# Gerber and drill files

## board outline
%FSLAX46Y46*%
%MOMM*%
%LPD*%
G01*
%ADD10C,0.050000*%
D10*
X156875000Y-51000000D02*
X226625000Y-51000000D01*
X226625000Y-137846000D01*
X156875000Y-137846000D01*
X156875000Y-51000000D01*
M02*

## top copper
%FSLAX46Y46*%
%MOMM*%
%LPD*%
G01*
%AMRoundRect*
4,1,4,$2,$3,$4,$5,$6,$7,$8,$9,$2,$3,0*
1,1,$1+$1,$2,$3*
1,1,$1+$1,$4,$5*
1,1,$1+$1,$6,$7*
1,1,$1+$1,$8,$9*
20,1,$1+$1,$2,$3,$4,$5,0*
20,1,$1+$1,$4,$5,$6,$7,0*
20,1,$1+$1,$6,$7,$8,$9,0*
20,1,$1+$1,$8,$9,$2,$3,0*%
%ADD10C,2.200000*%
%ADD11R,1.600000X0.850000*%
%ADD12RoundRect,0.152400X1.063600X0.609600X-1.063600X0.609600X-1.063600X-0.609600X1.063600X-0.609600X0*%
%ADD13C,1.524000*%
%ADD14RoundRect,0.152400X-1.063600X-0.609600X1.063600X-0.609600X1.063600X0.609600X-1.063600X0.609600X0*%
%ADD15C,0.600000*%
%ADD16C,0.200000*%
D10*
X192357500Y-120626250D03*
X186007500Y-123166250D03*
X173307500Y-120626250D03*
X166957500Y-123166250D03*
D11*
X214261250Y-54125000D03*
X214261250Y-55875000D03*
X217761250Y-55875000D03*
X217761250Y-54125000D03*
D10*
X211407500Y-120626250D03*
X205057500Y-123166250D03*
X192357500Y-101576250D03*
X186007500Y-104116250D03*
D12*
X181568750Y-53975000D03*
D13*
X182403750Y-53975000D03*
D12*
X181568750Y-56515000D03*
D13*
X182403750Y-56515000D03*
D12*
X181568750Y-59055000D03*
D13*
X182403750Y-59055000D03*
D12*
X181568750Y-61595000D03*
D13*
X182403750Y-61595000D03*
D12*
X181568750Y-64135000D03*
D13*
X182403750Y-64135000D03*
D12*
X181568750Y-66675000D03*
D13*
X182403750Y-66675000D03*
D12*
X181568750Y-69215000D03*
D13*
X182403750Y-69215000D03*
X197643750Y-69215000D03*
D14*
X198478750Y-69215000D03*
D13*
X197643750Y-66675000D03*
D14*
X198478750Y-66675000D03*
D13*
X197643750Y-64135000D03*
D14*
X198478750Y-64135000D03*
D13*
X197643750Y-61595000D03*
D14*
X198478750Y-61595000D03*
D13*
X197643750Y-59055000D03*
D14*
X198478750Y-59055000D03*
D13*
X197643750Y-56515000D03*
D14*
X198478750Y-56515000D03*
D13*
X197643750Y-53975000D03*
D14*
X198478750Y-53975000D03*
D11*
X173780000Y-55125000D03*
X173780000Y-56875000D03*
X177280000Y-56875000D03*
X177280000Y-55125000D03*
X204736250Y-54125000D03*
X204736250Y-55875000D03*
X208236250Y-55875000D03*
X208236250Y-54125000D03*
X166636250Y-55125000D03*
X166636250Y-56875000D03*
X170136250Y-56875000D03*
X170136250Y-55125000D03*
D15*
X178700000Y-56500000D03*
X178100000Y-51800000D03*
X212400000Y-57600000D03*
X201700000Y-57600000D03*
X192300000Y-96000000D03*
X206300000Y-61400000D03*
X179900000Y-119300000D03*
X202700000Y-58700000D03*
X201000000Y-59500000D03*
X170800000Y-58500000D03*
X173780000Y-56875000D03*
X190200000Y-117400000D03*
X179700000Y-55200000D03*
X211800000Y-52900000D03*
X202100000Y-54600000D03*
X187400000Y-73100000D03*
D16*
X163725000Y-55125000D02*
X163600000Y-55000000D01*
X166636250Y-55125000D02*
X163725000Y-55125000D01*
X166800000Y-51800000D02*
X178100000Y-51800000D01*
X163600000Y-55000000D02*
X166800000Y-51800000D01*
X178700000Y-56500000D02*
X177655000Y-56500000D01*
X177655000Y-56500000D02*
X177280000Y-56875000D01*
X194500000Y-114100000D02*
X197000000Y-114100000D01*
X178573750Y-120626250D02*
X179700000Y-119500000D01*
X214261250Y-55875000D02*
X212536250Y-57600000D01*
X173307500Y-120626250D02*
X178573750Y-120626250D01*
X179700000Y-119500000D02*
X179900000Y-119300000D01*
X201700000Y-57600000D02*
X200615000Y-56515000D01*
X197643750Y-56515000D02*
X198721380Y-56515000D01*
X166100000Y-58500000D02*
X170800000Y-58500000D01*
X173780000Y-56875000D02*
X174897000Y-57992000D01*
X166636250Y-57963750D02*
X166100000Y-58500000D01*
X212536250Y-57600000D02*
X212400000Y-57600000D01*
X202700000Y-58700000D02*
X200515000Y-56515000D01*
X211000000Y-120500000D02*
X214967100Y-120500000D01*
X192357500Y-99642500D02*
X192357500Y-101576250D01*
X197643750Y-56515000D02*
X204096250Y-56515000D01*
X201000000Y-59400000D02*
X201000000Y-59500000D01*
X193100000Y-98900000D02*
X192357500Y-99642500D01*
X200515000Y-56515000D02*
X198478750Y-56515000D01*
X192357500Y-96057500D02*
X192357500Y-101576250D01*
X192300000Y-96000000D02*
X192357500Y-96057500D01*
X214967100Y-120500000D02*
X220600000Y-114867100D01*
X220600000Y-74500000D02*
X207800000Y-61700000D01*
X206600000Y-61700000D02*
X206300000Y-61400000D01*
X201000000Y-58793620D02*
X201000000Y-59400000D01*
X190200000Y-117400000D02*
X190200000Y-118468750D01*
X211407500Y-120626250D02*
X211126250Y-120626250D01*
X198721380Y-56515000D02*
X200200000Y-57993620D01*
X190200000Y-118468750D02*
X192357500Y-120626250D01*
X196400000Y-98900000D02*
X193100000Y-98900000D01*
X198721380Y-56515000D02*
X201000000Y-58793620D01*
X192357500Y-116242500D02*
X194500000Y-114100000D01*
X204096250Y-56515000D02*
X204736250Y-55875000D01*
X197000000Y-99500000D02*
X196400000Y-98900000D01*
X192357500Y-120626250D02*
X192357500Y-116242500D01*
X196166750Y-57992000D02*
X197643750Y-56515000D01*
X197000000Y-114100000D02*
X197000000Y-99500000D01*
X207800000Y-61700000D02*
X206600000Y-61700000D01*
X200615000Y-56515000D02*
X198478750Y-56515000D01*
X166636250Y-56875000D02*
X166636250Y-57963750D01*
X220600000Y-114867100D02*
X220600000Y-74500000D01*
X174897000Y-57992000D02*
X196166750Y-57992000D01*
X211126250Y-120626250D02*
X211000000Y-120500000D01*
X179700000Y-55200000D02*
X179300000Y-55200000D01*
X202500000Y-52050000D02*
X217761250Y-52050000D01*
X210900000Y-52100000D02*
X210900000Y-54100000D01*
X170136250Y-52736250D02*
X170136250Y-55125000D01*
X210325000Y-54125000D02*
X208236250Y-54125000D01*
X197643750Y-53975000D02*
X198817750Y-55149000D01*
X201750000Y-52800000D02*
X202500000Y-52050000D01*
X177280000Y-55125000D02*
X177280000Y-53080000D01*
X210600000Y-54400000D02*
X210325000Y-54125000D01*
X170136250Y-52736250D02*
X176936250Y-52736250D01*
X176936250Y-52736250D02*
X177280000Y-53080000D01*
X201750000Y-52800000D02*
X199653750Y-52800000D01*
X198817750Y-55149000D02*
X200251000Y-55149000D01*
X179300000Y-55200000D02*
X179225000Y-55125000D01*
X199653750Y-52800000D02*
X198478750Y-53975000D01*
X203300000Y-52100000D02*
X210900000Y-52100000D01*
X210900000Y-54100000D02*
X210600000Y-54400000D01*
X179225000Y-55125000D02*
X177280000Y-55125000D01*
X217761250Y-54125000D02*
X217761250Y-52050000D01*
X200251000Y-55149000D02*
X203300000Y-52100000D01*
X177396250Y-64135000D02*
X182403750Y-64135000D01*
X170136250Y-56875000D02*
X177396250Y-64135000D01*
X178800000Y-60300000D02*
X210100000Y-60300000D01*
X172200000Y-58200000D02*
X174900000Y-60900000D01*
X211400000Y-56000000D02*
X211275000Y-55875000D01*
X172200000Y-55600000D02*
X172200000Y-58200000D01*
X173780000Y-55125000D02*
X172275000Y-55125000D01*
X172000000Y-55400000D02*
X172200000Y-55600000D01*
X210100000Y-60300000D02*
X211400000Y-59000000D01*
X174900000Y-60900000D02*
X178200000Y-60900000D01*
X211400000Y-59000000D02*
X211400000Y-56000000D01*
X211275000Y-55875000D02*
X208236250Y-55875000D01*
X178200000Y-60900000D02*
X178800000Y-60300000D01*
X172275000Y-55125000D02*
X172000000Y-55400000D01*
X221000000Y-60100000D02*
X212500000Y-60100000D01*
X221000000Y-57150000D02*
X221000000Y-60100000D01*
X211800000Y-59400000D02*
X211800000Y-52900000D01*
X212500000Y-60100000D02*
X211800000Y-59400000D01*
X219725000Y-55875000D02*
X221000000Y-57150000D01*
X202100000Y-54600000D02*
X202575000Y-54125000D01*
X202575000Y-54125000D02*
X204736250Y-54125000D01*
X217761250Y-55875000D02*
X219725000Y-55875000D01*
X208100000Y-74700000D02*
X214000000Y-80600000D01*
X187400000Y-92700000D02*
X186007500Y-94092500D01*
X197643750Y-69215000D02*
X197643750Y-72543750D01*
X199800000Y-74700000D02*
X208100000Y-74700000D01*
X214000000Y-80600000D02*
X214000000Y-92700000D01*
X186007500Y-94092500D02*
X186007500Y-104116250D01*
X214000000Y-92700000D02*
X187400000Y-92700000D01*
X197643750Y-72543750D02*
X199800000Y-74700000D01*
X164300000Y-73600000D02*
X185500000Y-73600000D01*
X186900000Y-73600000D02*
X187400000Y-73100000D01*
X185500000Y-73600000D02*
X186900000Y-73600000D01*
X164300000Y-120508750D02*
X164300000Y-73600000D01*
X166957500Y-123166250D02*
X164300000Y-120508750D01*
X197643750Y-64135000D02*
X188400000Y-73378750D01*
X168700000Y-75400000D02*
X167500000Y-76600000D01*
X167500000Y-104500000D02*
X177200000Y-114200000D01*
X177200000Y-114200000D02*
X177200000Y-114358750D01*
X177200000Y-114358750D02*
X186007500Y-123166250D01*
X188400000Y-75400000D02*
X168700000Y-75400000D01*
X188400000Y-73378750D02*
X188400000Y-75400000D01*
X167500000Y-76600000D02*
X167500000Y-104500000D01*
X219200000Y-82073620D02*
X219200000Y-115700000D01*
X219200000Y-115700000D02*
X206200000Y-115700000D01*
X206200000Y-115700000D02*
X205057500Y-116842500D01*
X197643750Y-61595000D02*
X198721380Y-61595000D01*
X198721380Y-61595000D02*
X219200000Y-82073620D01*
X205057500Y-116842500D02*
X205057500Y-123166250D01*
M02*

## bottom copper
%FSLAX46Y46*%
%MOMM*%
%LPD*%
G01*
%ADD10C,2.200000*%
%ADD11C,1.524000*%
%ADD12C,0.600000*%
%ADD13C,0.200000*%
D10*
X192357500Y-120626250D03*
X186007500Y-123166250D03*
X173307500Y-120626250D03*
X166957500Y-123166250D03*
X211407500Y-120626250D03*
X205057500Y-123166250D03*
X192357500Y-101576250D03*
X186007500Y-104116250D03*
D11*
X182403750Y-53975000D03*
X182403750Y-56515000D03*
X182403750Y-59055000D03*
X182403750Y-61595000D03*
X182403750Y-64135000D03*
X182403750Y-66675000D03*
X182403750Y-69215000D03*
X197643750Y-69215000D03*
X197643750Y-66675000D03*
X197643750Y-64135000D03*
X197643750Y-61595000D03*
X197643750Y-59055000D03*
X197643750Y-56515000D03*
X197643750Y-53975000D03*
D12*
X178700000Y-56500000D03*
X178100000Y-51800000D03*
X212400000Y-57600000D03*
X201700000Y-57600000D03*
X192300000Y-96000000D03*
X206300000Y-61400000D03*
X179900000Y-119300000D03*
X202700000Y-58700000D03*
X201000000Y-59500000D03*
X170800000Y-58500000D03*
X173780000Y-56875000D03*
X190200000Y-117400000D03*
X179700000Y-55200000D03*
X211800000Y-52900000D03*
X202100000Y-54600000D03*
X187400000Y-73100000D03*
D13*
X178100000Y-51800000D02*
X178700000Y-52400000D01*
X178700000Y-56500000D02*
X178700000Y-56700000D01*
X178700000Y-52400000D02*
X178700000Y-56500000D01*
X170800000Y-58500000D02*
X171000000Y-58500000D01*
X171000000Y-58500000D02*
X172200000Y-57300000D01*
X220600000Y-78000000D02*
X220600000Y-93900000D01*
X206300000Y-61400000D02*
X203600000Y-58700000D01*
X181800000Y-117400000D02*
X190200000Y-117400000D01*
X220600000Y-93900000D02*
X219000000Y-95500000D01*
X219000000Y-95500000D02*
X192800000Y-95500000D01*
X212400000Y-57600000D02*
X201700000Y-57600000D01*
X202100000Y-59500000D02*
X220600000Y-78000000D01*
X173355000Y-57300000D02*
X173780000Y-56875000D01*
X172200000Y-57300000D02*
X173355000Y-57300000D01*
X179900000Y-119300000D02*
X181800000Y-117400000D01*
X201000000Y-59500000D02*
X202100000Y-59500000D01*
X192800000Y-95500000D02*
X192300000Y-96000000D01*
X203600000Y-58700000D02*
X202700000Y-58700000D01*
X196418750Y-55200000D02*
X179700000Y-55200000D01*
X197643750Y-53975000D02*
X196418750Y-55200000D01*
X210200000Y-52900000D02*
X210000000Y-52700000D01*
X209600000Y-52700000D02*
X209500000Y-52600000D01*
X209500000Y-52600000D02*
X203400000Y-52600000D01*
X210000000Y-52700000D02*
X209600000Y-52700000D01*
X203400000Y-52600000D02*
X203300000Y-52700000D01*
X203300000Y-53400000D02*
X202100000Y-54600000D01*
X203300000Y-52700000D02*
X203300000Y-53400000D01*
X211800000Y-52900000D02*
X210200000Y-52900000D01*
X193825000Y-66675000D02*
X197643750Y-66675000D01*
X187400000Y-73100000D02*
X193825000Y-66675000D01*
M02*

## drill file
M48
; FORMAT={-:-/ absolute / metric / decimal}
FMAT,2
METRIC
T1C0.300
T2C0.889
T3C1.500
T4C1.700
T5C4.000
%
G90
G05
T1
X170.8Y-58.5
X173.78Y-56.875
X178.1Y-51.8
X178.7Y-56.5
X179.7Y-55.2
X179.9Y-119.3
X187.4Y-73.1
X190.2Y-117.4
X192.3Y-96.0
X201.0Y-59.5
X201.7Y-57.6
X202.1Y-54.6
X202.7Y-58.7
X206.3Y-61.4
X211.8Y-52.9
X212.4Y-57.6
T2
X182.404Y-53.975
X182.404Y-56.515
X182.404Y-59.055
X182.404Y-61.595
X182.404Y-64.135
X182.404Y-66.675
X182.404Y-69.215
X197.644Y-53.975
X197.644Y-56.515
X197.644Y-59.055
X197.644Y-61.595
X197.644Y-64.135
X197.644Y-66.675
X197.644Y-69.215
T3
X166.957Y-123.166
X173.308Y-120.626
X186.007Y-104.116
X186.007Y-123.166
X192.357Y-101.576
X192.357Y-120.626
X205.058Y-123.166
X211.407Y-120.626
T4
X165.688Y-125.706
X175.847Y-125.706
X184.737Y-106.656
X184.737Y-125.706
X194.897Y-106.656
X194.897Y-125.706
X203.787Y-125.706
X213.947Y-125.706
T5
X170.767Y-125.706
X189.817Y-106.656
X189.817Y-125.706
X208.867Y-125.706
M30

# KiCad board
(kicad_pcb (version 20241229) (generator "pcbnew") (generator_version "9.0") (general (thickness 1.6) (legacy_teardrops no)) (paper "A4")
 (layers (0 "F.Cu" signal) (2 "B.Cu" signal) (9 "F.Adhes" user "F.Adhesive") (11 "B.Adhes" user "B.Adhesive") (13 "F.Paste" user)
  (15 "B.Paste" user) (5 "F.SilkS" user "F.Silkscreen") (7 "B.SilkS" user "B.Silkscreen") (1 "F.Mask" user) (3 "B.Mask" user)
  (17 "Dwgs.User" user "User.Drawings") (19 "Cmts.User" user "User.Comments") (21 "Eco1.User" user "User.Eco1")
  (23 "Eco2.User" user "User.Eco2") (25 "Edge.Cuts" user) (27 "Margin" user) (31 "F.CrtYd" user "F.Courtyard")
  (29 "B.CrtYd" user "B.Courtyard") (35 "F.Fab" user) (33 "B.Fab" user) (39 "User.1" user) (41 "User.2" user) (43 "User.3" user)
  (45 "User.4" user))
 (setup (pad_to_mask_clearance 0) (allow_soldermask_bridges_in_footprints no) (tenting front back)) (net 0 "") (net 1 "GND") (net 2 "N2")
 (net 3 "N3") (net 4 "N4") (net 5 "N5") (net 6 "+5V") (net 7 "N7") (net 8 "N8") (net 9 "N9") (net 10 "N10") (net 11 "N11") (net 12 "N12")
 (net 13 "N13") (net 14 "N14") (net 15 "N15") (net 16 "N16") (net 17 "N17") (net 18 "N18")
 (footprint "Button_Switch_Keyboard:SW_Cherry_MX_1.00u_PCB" (layer "F.Cu") (at 192.3575 120.62625)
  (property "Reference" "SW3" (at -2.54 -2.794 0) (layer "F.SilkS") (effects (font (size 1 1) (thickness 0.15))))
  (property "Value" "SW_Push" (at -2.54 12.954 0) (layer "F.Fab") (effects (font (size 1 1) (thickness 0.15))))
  (pad "" np_thru_hole circle (at -7.62 5.08) (size 1.7 1.7) (drill 1.7) (layers "*.Cu" "*.Mask"))
  (pad "" np_thru_hole circle (at -2.54 5.08) (size 4 4) (drill 4) (layers "*.Cu" "*.Mask"))
  (pad "" np_thru_hole circle (at 2.54 5.08) (size 1.7 1.7) (drill 1.7) (layers "*.Cu" "*.Mask"))
  (pad "1" thru_hole circle (at 0 0) (size 2.2 2.2) (drill 1.5) (layers "*.Cu" "*.Mask") (remove_unused_layers no) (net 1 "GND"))
  (pad "2" thru_hole circle (at -6.35 2.54) (size 2.2 2.2) (drill 1.5) (layers "*.Cu" "*.Mask") (remove_unused_layers no) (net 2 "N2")))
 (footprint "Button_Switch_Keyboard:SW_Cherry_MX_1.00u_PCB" (layer "F.Cu") (at 173.3075 120.62625)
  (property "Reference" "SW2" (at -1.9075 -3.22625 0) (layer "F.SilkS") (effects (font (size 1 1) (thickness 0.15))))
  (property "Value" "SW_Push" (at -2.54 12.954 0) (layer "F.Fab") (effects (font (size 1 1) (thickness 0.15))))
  (pad "" np_thru_hole circle (at -7.62 5.08) (size 1.7 1.7) (drill 1.7) (layers "*.Cu" "*.Mask"))
  (pad "" np_thru_hole circle (at -2.54 5.08) (size 4 4) (drill 4) (layers "*.Cu" "*.Mask"))
  (pad "" np_thru_hole circle (at 2.54 5.08) (size 1.7 1.7) (drill 1.7) (layers "*.Cu" "*.Mask"))
  (pad "1" thru_hole circle (at 0 0) (size 2.2 2.2) (drill 1.5) (layers "*.Cu" "*.Mask") (remove_unused_layers no) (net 1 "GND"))
  (pad "2" thru_hole circle (at -6.35 2.54) (size 2.2 2.2) (drill 1.5) (layers "*.Cu" "*.Mask") (remove_unused_layers no) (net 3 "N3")))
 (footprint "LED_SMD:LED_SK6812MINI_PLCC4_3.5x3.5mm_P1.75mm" (layer "F.Cu") (at 216.01125 55)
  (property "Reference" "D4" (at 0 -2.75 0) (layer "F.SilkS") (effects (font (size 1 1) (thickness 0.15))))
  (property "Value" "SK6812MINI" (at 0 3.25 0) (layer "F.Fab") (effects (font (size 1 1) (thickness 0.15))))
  (pad "1" smd rect (at -1.75 -0.875) (size 1.6 0.85) (layers "F.Cu" "F.Mask" "F.Paste") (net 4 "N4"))
  (pad "2" smd rect (at -1.75 0.875) (size 1.6 0.85) (layers "F.Cu" "F.Mask" "F.Paste") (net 1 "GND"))
  (pad "3" smd rect (at 1.75 0.875) (size 1.6 0.85) (layers "F.Cu" "F.Mask" "F.Paste") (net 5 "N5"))
  (pad "4" smd rect (at 1.75 -0.875) (size 1.6 0.85) (layers "F.Cu" "F.Mask" "F.Paste") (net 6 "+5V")))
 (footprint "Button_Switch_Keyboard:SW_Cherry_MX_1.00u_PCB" (layer "F.Cu") (at 211.4075 120.62625)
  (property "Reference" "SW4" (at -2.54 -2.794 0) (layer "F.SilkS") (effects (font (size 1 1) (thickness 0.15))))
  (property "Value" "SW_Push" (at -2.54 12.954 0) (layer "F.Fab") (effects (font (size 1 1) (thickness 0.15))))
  (pad "" np_thru_hole circle (at -7.62 5.08) (size 1.7 1.7) (drill 1.7) (layers "*.Cu" "*.Mask"))
  (pad "" np_thru_hole circle (at -2.54 5.08) (size 4 4) (drill 4) (layers "*.Cu" "*.Mask"))
  (pad "" np_thru_hole circle (at 2.54 5.08) (size 1.7 1.7) (drill 1.7) (layers "*.Cu" "*.Mask"))
  (pad "1" thru_hole circle (at 0 0) (size 2.2 2.2) (drill 1.5) (layers "*.Cu" "*.Mask") (remove_unused_layers no) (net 1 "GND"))
  (pad "2" thru_hole circle (at -6.35 2.54) (size 2.2 2.2) (drill 1.5) (layers "*.Cu" "*.Mask") (remove_unused_layers no) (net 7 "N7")))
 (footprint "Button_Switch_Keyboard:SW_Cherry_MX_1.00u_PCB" (layer "F.Cu") (at 192.3575 101.57625)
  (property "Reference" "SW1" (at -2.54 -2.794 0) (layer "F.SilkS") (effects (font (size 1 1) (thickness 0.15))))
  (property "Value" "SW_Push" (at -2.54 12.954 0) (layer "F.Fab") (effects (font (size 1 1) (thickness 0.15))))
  (pad "" np_thru_hole circle (at -7.62 5.08) (size 1.7 1.7) (drill 1.7) (layers "*.Cu" "*.Mask"))
  (pad "" np_thru_hole circle (at -2.54 5.08) (size 4 4) (drill 4) (layers "*.Cu" "*.Mask"))
  (pad "" np_thru_hole circle (at 2.54 5.08) (size 1.7 1.7) (drill 1.7) (layers "*.Cu" "*.Mask"))
  (pad "1" thru_hole circle (at 0 0) (size 2.2 2.2) (drill 1.5) (layers "*.Cu" "*.Mask") (remove_unused_layers no) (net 1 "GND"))
  (pad "2" thru_hole circle (at -6.35 2.54) (size 2.2 2.2) (drill 1.5) (layers "*.Cu" "*.Mask") (remove_unused_layers no) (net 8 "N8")))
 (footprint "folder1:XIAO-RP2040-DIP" (layer "F.Cu") (at 190.02375 61.595)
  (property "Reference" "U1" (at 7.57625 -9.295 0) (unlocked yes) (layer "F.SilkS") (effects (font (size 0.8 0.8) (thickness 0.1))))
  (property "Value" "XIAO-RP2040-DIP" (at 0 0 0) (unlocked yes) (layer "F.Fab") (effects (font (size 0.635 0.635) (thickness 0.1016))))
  (pad "1" smd roundrect (at -8.455 -7.62 180) (size 2.432 1.524) (layers "F.Cu" "F.Mask") (roundrect_rratio 0.1) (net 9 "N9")
   (thermal_bridge_angle 45))
  (pad "1" thru_hole circle (at -7.62 -7.62 180) (size 1.524 1.524) (drill 0.889) (layers "*.Cu" "*.Mask") (remove_unused_layers no)
   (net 9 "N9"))
  (pad "2" smd roundrect (at -8.455 -5.08 180) (size 2.432 1.524) (layers "F.Cu" "F.Mask") (roundrect_rratio 0.1) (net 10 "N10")
   (thermal_bridge_angle 45))
  (pad "2" thru_hole circle (at -7.62 -5.08 180) (size 1.524 1.524) (drill 0.889) (layers "*.Cu" "*.Mask") (remove_unused_layers no)
   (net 10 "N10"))
  (pad "3" smd roundrect (at -8.455 -2.54 180) (size 2.432 1.524) (layers "F.Cu" "F.Mask") (roundrect_rratio 0.1) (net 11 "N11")
   (thermal_bridge_angle 45))
  (pad "3" thru_hole circle (at -7.62 -2.54 180) (size 1.524 1.524) (drill 0.889) (layers "*.Cu" "*.Mask") (remove_unused_layers no)
   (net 11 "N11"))
  (pad "4" smd roundrect (at -8.455 0 180) (size 2.432 1.524) (layers "F.Cu" "F.Mask") (roundrect_rratio 0.1) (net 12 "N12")
   (thermal_bridge_angle 45))
  (pad "4" thru_hole circle (at -7.62 0 180) (size 1.524 1.524) (drill 0.889) (layers "*.Cu" "*.Mask") (remove_unused_layers no)
   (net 12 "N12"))
  (pad "5" smd roundrect (at -8.455 2.54 180) (size 2.432 1.524) (layers "F.Cu" "F.Mask") (roundrect_rratio 0.1) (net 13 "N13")
   (thermal_bridge_angle 45))
  (pad "5" thru_hole circle (at -7.62 2.54 180) (size 1.524 1.524) (drill 0.889) (layers "*.Cu" "*.Mask") (remove_unused_layers no)
   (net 13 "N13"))
  (pad "6" smd roundrect (at -8.455 5.08 180) (size 2.432 1.524) (layers "F.Cu" "F.Mask") (roundrect_rratio 0.1) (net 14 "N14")
   (thermal_bridge_angle 45))
  (pad "6" thru_hole circle (at -7.62 5.08 180) (size 1.524 1.524) (drill 0.889) (layers "*.Cu" "*.Mask") (remove_unused_layers no)
   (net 14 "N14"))
  (pad "7" smd roundrect (at -8.455 7.62 180) (size 2.432 1.524) (layers "F.Cu" "F.Mask") (roundrect_rratio 0.1) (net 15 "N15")
   (thermal_bridge_angle 45))
  (pad "7" thru_hole circle (at -7.62 7.62 180) (size 1.524 1.524) (drill 0.889) (layers "*.Cu" "*.Mask") (remove_unused_layers no)
   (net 15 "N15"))
  (pad "8" thru_hole circle (at 7.62 7.62) (size 1.524 1.524) (drill 0.889) (layers "*.Cu" "*.Mask") (remove_unused_layers no) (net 8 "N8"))
  (pad "8" smd roundrect (at 8.455 7.62) (size 2.432 1.524) (layers "F.Cu" "F.Mask") (roundrect_rratio 0.1) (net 8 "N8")
   (thermal_bridge_angle 45))
  (pad "9" thru_hole circle (at 7.62 5.08) (size 1.524 1.524) (drill 0.889) (layers "*.Cu" "*.Mask") (remove_unused_layers no) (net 3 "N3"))
  (pad "9" smd roundrect (at 8.455 5.08) (size 2.432 1.524) (layers "F.Cu" "F.Mask") (roundrect_rratio 0.1) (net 3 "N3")
   (thermal_bridge_angle 45))
  (pad "10" thru_hole circle (at 7.62 2.54) (size 1.524 1.524) (drill 0.889) (layers "*.Cu" "*.Mask") (remove_unused_layers no) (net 2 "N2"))
  (pad "10" smd roundrect (at 8.455 2.54) (size 2.432 1.524) (layers "F.Cu" "F.Mask") (roundrect_rratio 0.1) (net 2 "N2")
   (thermal_bridge_angle 45))
  (pad "11" thru_hole circle (at 7.62 0) (size 1.524 1.524) (drill 0.889) (layers "*.Cu" "*.Mask") (remove_unused_layers no) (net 7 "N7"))
  (pad "11" smd roundrect (at 8.455 0) (size 2.432 1.524) (layers "F.Cu" "F.Mask") (roundrect_rratio 0.1) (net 7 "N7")
   (thermal_bridge_angle 45))
  (pad "12" thru_hole circle (at 7.62 -2.54) (size 1.524 1.524) (drill 0.889) (layers "*.Cu" "*.Mask") (remove_unused_layers no)
   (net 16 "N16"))
  (pad "12" smd roundrect (at 8.455 -2.54) (size 2.432 1.524) (layers "F.Cu" "F.Mask") (roundrect_rratio 0.1) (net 16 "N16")
   (thermal_bridge_angle 45))
  (pad "13" thru_hole circle (at 7.62 -5.08) (size 1.524 1.524) (drill 0.889) (layers "*.Cu" "*.Mask") (remove_unused_layers no)
   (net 1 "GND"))
  (pad "13" smd roundrect (at 8.455 -5.08) (size 2.432 1.524) (layers "F.Cu" "F.Mask") (roundrect_rratio 0.1) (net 1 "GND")
   (thermal_bridge_angle 45))
  (pad "14" thru_hole circle (at 7.62 -7.62) (size 1.524 1.524) (drill 0.889) (layers "*.Cu" "*.Mask") (remove_unused_layers no)
   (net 6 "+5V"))
  (pad "14" smd roundrect (at 8.455 -7.62) (size 2.432 1.524) (layers "F.Cu" "F.Mask") (roundrect_rratio 0.1) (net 6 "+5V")
   (thermal_bridge_angle 45)))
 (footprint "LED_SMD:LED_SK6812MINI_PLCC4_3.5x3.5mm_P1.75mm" (layer "F.Cu") (at 175.53 56)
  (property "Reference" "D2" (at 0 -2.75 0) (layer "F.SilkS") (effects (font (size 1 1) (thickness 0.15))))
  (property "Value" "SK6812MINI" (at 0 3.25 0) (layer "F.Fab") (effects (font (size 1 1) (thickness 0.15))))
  (pad "1" smd rect (at -1.75 -0.875) (size 1.6 0.85) (layers "F.Cu" "F.Mask" "F.Paste") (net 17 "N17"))
  (pad "2" smd rect (at -1.75 0.875) (size 1.6 0.85) (layers "F.Cu" "F.Mask" "F.Paste") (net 1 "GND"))
  (pad "3" smd rect (at 1.75 0.875) (size 1.6 0.85) (layers "F.Cu" "F.Mask" "F.Paste") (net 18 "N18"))
  (pad "4" smd rect (at 1.75 -0.875) (size 1.6 0.85) (layers "F.Cu" "F.Mask" "F.Paste") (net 6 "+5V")))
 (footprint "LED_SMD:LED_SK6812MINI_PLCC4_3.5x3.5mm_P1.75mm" (layer "F.Cu") (at 206.48625 55)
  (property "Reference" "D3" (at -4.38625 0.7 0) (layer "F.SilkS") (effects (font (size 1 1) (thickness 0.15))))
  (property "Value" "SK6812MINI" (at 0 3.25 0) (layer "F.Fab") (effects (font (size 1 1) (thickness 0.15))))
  (pad "1" smd rect (at -1.75 -0.875) (size 1.6 0.85) (layers "F.Cu" "F.Mask" "F.Paste") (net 5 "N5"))
  (pad "2" smd rect (at -1.75 0.875) (size 1.6 0.85) (layers "F.Cu" "F.Mask" "F.Paste") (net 1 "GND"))
  (pad "3" smd rect (at 1.75 0.875) (size 1.6 0.85) (layers "F.Cu" "F.Mask" "F.Paste") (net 17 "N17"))
  (pad "4" smd rect (at 1.75 -0.875) (size 1.6 0.85) (layers "F.Cu" "F.Mask" "F.Paste") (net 6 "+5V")))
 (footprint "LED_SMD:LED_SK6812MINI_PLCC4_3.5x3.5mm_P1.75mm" (layer "F.Cu") (at 168.38625 56)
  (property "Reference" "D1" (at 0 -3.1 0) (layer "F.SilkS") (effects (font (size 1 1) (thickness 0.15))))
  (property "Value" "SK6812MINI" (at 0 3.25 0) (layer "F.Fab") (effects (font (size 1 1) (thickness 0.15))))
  (pad "1" smd rect (at -1.75 -0.875) (size 1.6 0.85) (layers "F.Cu" "F.Mask" "F.Paste") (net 18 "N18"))
  (pad "2" smd rect (at -1.75 0.875) (size 1.6 0.85) (layers "F.Cu" "F.Mask" "F.Paste") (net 1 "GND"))
  (pad "3" smd rect (at 1.75 0.875) (size 1.6 0.85) (layers "F.Cu" "F.Mask" "F.Paste") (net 13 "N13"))
  (pad "4" smd rect (at 1.75 -0.875) (size 1.6 0.85) (layers "F.Cu" "F.Mask" "F.Paste") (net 6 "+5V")))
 (gr_rect (start 156.875 51) (end 226.625 137.846) (stroke (width 0.05) (type default)) (fill no) (layer "Edge.Cuts"))
 (segment (start 163.725 55.125) (end 163.6 55) (width 0.2) (layer "F.Cu") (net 18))
 (segment (start 166.63625 55.125) (end 163.725 55.125) (width 0.2) (layer "F.Cu") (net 18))
 (segment (start 166.8 51.8) (end 178.1 51.8) (width 0.2) (layer "F.Cu") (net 18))
 (segment (start 163.6 55) (end 166.8 51.8) (width 0.2) (layer "F.Cu") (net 18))
 (segment (start 178.7 56.5) (end 177.655 56.5) (width 0.2) (layer "F.Cu") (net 18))
 (segment (start 177.655 56.5) (end 177.28 56.875) (width 0.2) (layer "F.Cu") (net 18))
 (via (at 178.7 56.5) (size 0.6) (drill 0.3) (layers "F.Cu" "B.Cu") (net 18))
 (via (at 178.1 51.8) (size 0.6) (drill 0.3) (layers "F.Cu" "B.Cu") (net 18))
 (segment (start 178.1 51.8) (end 178.7 52.4) (width 0.2) (layer "B.Cu") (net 18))
 (segment (start 178.7 56.5) (end 178.7 56.7) (width 0.2) (layer "B.Cu") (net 18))
 (segment (start 178.7 52.4) (end 178.7 56.5) (width 0.2) (layer "B.Cu") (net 18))
 (segment (start 194.5 114.1) (end 197 114.1) (width 0.2) (layer "F.Cu") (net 1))
 (segment (start 178.57375 120.62625) (end 179.7 119.5) (width 0.2) (layer "F.Cu") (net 1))
 (segment (start 214.26125 55.875) (end 212.53625 57.6) (width 0.2) (layer "F.Cu") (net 1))
 (segment (start 173.3075 120.62625) (end 178.57375 120.62625) (width 0.2) (layer "F.Cu") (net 1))
 (segment (start 179.7 119.5) (end 179.9 119.3) (width 0.2) (layer "F.Cu") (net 1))
 (segment (start 201.7 57.6) (end 200.615 56.515) (width 0.2) (layer "F.Cu") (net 1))
 (segment (start 197.64375 56.515) (end 198.72138 56.515) (width 0.2) (layer "F.Cu") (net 1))
 (segment (start 166.1 58.5) (end 170.8 58.5) (width 0.2) (layer "F.Cu") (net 1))
 (segment (start 173.78 56.875) (end 174.897 57.992) (width 0.2) (layer "F.Cu") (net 1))
 (segment (start 166.63625 57.96375) (end 166.1 58.5) (width 0.2) (layer "F.Cu") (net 1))
 (segment (start 212.53625 57.6) (end 212.4 57.6) (width 0.2) (layer "F.Cu") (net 1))
 (segment (start 202.7 58.7) (end 200.515 56.515) (width 0.2) (layer "F.Cu") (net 1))
 (segment (start 211 120.5) (end 214.9671 120.5) (width 0.2) (layer "F.Cu") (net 1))
 (segment (start 192.3575 99.6425) (end 192.3575 101.57625) (width 0.2) (layer "F.Cu") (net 1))
 (segment (start 197.64375 56.515) (end 204.09625 56.515) (width 0.2) (layer "F.Cu") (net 1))
 (segment (start 201 59.4) (end 201 59.5) (width 0.2) (layer "F.Cu") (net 1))
 (segment (start 193.1 98.9) (end 192.3575 99.6425) (width 0.2) (layer "F.Cu") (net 1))
 (segment (start 200.515 56.515) (end 198.47875 56.515) (width 0.2) (layer "F.Cu") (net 1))
 (segment (start 192.3575 96.0575) (end 192.3575 101.57625) (width 0.2) (layer "F.Cu") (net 1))
 (segment (start 192.3 96) (end 192.3575 96.0575) (width 0.2) (layer "F.Cu") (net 1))
 (segment (start 214.9671 120.5) (end 220.6 114.8671) (width 0.2) (layer "F.Cu") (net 1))
 (segment (start 220.6 74.5) (end 207.8 61.7) (width 0.2) (layer "F.Cu") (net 1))
 (segment (start 206.6 61.7) (end 206.3 61.4) (width 0.2) (layer "F.Cu") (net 1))
 (segment (start 201 58.79362) (end 201 59.4) (width 0.2) (layer "F.Cu") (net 1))
 (segment (start 190.2 117.4) (end 190.2 118.46875) (width 0.2) (layer "F.Cu") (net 1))
 (segment (start 211.4075 120.62625) (end 211.12625 120.62625) (width 0.2) (layer "F.Cu") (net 1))
 (segment (start 198.72138 56.515) (end 200.2 57.99362) (width 0.2) (layer "F.Cu") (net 1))
 (segment (start 190.2 118.46875) (end 192.3575 120.62625) (width 0.2) (layer "F.Cu") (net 1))
 (segment (start 196.4 98.9) (end 193.1 98.9) (width 0.2) (layer "F.Cu") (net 1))
 (segment (start 198.72138 56.515) (end 201 58.79362) (width 0.2) (layer "F.Cu") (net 1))
 (segment (start 192.3575 116.2425) (end 194.5 114.1) (width 0.2) (layer "F.Cu") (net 1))
 (segment (start 204.09625 56.515) (end 204.73625 55.875) (width 0.2) (layer "F.Cu") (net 1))
 (segment (start 197 99.5) (end 196.4 98.9) (width 0.2) (layer "F.Cu") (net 1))
 (segment (start 192.3575 120.62625) (end 192.3575 116.2425) (width 0.2) (layer "F.Cu") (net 1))
 (segment (start 196.16675 57.992) (end 197.64375 56.515) (width 0.2) (layer "F.Cu") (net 1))
 (segment (start 197 114.1) (end 197 99.5) (width 0.2) (layer "F.Cu") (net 1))
 (segment (start 207.8 61.7) (end 206.6 61.7) (width 0.2) (layer "F.Cu") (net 1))
 (segment (start 200.615 56.515) (end 198.47875 56.515) (width 0.2) (layer "F.Cu") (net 1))
 (segment (start 166.63625 56.875) (end 166.63625 57.96375) (width 0.2) (layer "F.Cu") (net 1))
 (segment (start 220.6 114.8671) (end 220.6 74.5) (width 0.2) (layer "F.Cu") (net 1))
 (segment (start 174.897 57.992) (end 196.16675 57.992) (width 0.2) (layer "F.Cu") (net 1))
 (segment (start 211.12625 120.62625) (end 211 120.5) (width 0.2) (layer "F.Cu") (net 1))
 (via (at 212.4 57.6) (size 0.6) (drill 0.3) (layers "F.Cu" "B.Cu") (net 1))
 (via (at 201.7 57.6) (size 0.6) (drill 0.3) (layers "F.Cu" "B.Cu") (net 1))
 (via (at 192.3 96) (size 0.6) (drill 0.3) (layers "F.Cu" "B.Cu") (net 1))
 (via (at 206.3 61.4) (size 0.6) (drill 0.3) (layers "F.Cu" "B.Cu") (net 1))
 (via (at 179.9 119.3) (size 0.6) (drill 0.3) (layers "F.Cu" "B.Cu") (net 1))
 (via (at 202.7 58.7) (size 0.6) (drill 0.3) (layers "F.Cu" "B.Cu") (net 1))
 (via (at 201 59.5) (size 0.6) (drill 0.3) (layers "F.Cu" "B.Cu") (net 1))
 (via (at 170.8 58.5) (size 0.6) (drill 0.3) (layers "F.Cu" "B.Cu") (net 1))
 (via (at 173.78 56.875) (size 0.6) (drill 0.3) (layers "F.Cu" "B.Cu") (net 1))
 (via (at 190.2 117.4) (size 0.6) (drill 0.3) (layers "F.Cu" "B.Cu") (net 1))
 (segment (start 170.8 58.5) (end 171 58.5) (width 0.2) (layer "B.Cu") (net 1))
 (segment (start 171 58.5) (end 172.2 57.3) (width 0.2) (layer "B.Cu") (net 1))
 (segment (start 220.6 78) (end 220.6 93.9) (width 0.2) (layer "B.Cu") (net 1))
 (segment (start 206.3 61.4) (end 203.6 58.7) (width 0.2) (layer "B.Cu") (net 1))
 (segment (start 181.8 117.4) (end 190.2 117.4) (width 0.2) (layer "B.Cu") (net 1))
 (segment (start 220.6 93.9) (end 219 95.5) (width 0.2) (layer "B.Cu") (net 1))
 (segment (start 219 95.5) (end 192.8 95.5) (width 0.2) (layer "B.Cu") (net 1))
 (segment (start 212.4 57.6) (end 201.7 57.6) (width 0.2) (layer "B.Cu") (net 1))
 (segment (start 202.1 59.5) (end 220.6 78) (width 0.2) (layer "B.Cu") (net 1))
 (segment (start 173.355 57.3) (end 173.78 56.875) (width 0.2) (layer "B.Cu") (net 1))
 (segment (start 172.2 57.3) (end 173.355 57.3) (width 0.2) (layer "B.Cu") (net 1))
 (segment (start 179.9 119.3) (end 181.8 117.4) (width 0.2) (layer "B.Cu") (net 1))
 (segment (start 201 59.5) (end 202.1 59.5) (width 0.2) (layer "B.Cu") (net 1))
 (segment (start 192.8 95.5) (end 192.3 96) (width 0.2) (layer "B.Cu") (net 1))
 (segment (start 203.6 58.7) (end 202.7 58.7) (width 0.2) (layer "B.Cu") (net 1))
 (segment (start 179.7 55.2) (end 179.3 55.2) (width 0.2) (layer "F.Cu") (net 6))
 (segment (start 202.5 52.05) (end 217.76125 52.05) (width 0.2) (layer "F.Cu") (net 6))
 (segment (start 210.9 52.1) (end 210.9 54.1) (width 0.2) (layer "F.Cu") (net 6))
 (segment (start 170.13625 52.73625) (end 170.13625 55.125) (width 0.2) (layer "F.Cu") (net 6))
 (segment (start 210.325 54.125) (end 208.23625 54.125) (width 0.2) (layer "F.Cu") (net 6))
 (segment (start 197.64375 53.975) (end 198.81775 55.149) (width 0.2) (layer "F.Cu") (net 6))
 (segment (start 201.75 52.8) (end 202.5 52.05) (width 0.2) (layer "F.Cu") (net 6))
 (segment (start 177.28 55.125) (end 177.28 53.08) (width 0.2) (layer "F.Cu") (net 6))
 (segment (start 210.6 54.4) (end 210.325 54.125) (width 0.2) (layer "F.Cu") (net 6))
 (segment (start 170.13625 52.73625) (end 176.93625 52.73625) (width 0.2) (layer "F.Cu") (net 6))
 (segment (start 176.93625 52.73625) (end 177.28 53.08) (width 0.2) (layer "F.Cu") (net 6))
 (segment (start 201.75 52.8) (end 199.65375 52.8) (width 0.2) (layer "F.Cu") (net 6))
 (segment (start 198.81775 55.149) (end 200.251 55.149) (width 0.2) (layer "F.Cu") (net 6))
 (segment (start 179.3 55.2) (end 179.225 55.125) (width 0.2) (layer "F.Cu") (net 6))
 (segment (start 199.65375 52.8) (end 198.47875 53.975) (width 0.2) (layer "F.Cu") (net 6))
 (segment (start 203.3 52.1) (end 210.9 52.1) (width 0.2) (layer "F.Cu") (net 6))
 (segment (start 210.9 54.1) (end 210.6 54.4) (width 0.2) (layer "F.Cu") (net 6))
 (segment (start 179.225 55.125) (end 177.28 55.125) (width 0.2) (layer "F.Cu") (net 6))
 (segment (start 217.76125 54.125) (end 217.76125 52.05) (width 0.2) (layer "F.Cu") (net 6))
 (segment (start 200.251 55.149) (end 203.3 52.1) (width 0.2) (layer "F.Cu") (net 6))
 (via (at 179.7 55.2) (size 0.6) (drill 0.3) (layers "F.Cu" "B.Cu") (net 6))
 (segment (start 196.41875 55.2) (end 179.7 55.2) (width 0.2) (layer "B.Cu") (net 6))
 (segment (start 197.64375 53.975) (end 196.41875 55.2) (width 0.2) (layer "B.Cu") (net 6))
 (segment (start 177.39625 64.135) (end 182.40375 64.135) (width 0.2) (layer "F.Cu") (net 13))
 (segment (start 170.13625 56.875) (end 177.39625 64.135) (width 0.2) (layer "F.Cu") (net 13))
 (segment (start 178.8 60.3) (end 210.1 60.3) (width 0.2) (layer "F.Cu") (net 17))
 (segment (start 172.2 58.2) (end 174.9 60.9) (width 0.2) (layer "F.Cu") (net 17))
 (segment (start 211.4 56) (end 211.275 55.875) (width 0.2) (layer "F.Cu") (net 17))
 (segment (start 172.2 55.6) (end 172.2 58.2) (width 0.2) (layer "F.Cu") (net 17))
 (segment (start 173.78 55.125) (end 172.275 55.125) (width 0.2) (layer "F.Cu") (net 17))
 (segment (start 172 55.4) (end 172.2 55.6) (width 0.2) (layer "F.Cu") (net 17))
 (segment (start 210.1 60.3) (end 211.4 59) (width 0.2) (layer "F.Cu") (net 17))
 (segment (start 174.9 60.9) (end 178.2 60.9) (width 0.2) (layer "F.Cu") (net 17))
 (segment (start 211.4 59) (end 211.4 56) (width 0.2) (layer "F.Cu") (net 17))
 (segment (start 211.275 55.875) (end 208.23625 55.875) (width 0.2) (layer "F.Cu") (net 17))
 (segment (start 178.2 60.9) (end 178.8 60.3) (width 0.2) (layer "F.Cu") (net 17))
 (segment (start 172.275 55.125) (end 172 55.4) (width 0.2) (layer "F.Cu") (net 17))
 (segment (start 221 60.1) (end 212.5 60.1) (width 0.2) (layer "F.Cu") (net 5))
 (segment (start 221 57.15) (end 221 60.1) (width 0.2) (layer "F.Cu") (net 5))
 (segment (start 211.8 59.4) (end 211.8 52.9) (width 0.2) (layer "F.Cu") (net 5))
 (segment (start 212.5 60.1) (end 211.8 59.4) (width 0.2) (layer "F.Cu") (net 5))
 (segment (start 219.725 55.875) (end 221 57.15) (width 0.2) (layer "F.Cu") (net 5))
 (segment (start 202.1 54.6) (end 202.575 54.125) (width 0.2) (layer "F.Cu") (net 5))
 (segment (start 202.575 54.125) (end 204.73625 54.125) (width 0.2) (layer "F.Cu") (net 5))
 (segment (start 217.76125 55.875) (end 219.725 55.875) (width 0.2) (layer "F.Cu") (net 5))
 (via (at 211.8 52.9) (size 0.6) (drill 0.3) (layers "F.Cu" "B.Cu") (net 5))
 (via (at 202.1 54.6) (size 0.6) (drill 0.3) (layers "F.Cu" "B.Cu") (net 5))
 (segment (start 210.2 52.9) (end 210 52.7) (width 0.2) (layer "B.Cu") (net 5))
 (segment (start 209.6 52.7) (end 209.5 52.6) (width 0.2) (layer "B.Cu") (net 5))
 (segment (start 209.5 52.6) (end 203.4 52.6) (width 0.2) (layer "B.Cu") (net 5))
 (segment (start 210 52.7) (end 209.6 52.7) (width 0.2) (layer "B.Cu") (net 5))
 (segment (start 203.4 52.6) (end 203.3 52.7) (width 0.2) (layer "B.Cu") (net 5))
 (segment (start 203.3 53.4) (end 202.1 54.6) (width 0.2) (layer "B.Cu") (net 5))
 (segment (start 203.3 52.7) (end 203.3 53.4) (width 0.2) (layer "B.Cu") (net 5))
 (segment (start 211.8 52.9) (end 210.2 52.9) (width 0.2) (layer "B.Cu") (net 5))
 (segment (start 208.1 74.7) (end 214 80.6) (width 0.2) (layer "F.Cu") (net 8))
 (segment (start 187.4 92.7) (end 186.0075 94.0925) (width 0.2) (layer "F.Cu") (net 8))
 (segment (start 197.64375 69.215) (end 197.64375 72.54375) (width 0.2) (layer "F.Cu") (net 8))
 (segment (start 199.8 74.7) (end 208.1 74.7) (width 0.2) (layer "F.Cu") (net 8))
 (segment (start 214 80.6) (end 214 92.7) (width 0.2) (layer "F.Cu") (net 8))
 (segment (start 186.0075 94.0925) (end 186.0075 104.11625) (width 0.2) (layer "F.Cu") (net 8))
 (segment (start 214 92.7) (end 187.4 92.7) (width 0.2) (layer "F.Cu") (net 8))
 (segment (start 197.64375 72.54375) (end 199.8 74.7) (width 0.2) (layer "F.Cu") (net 8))
 (segment (start 164.3 73.6) (end 185.5 73.6) (width 0.2) (layer "F.Cu") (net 3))
 (segment (start 186.9 73.6) (end 187.4 73.1) (width 0.2) (layer "F.Cu") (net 3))
 (segment (start 185.5 73.6) (end 186.9 73.6) (width 0.2) (layer "F.Cu") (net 3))
 (segment (start 164.3 120.50875) (end 164.3 73.6) (width 0.2) (layer "F.Cu") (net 3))
 (segment (start 166.9575 123.16625) (end 164.3 120.50875) (width 0.2) (layer "F.Cu") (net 3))
 (via (at 187.4 73.1) (size 0.6) (drill 0.3) (layers "F.Cu" "B.Cu") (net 3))
 (segment (start 193.825 66.675) (end 197.64375 66.675) (width 0.2) (layer "B.Cu") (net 3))
 (segment (start 187.4 73.1) (end 193.825 66.675) (width 0.2) (layer "B.Cu") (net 3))
 (segment (start 197.64375 64.135) (end 188.4 73.37875) (width 0.2) (layer "F.Cu") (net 2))
 (segment (start 168.7 75.4) (end 167.5 76.6) (width 0.2) (layer "F.Cu") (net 2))
 (segment (start 167.5 104.5) (end 177.2 114.2) (width 0.2) (layer "F.Cu") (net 2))
 (segment (start 177.2 114.2) (end 177.2 114.35875) (width 0.2) (layer "F.Cu") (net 2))
 (segment (start 177.2 114.35875) (end 186.0075 123.16625) (width 0.2) (layer "F.Cu") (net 2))
 (segment (start 188.4 75.4) (end 168.7 75.4) (width 0.2) (layer "F.Cu") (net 2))
 (segment (start 188.4 73.37875) (end 188.4 75.4) (width 0.2) (layer "F.Cu") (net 2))
 (segment (start 167.5 76.6) (end 167.5 104.5) (width 0.2) (layer "F.Cu") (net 2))
 (segment (start 219.2 82.07362) (end 219.2 115.7) (width 0.2) (layer "F.Cu") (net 7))
 (segment (start 219.2 115.7) (end 206.2 115.7) (width 0.2) (layer "F.Cu") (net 7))
 (segment (start 206.2 115.7) (end 205.0575 116.8425) (width 0.2) (layer "F.Cu") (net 7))
 (segment (start 197.64375 61.595) (end 198.72138 61.595) (width 0.2) (layer "F.Cu") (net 7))
 (segment (start 198.72138 61.595) (end 219.2 82.07362) (width 0.2) (layer "F.Cu") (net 7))
 (segment (start 205.0575 116.8425) (end 205.0575 123.16625) (width 0.2) (layer "F.Cu") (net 7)))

